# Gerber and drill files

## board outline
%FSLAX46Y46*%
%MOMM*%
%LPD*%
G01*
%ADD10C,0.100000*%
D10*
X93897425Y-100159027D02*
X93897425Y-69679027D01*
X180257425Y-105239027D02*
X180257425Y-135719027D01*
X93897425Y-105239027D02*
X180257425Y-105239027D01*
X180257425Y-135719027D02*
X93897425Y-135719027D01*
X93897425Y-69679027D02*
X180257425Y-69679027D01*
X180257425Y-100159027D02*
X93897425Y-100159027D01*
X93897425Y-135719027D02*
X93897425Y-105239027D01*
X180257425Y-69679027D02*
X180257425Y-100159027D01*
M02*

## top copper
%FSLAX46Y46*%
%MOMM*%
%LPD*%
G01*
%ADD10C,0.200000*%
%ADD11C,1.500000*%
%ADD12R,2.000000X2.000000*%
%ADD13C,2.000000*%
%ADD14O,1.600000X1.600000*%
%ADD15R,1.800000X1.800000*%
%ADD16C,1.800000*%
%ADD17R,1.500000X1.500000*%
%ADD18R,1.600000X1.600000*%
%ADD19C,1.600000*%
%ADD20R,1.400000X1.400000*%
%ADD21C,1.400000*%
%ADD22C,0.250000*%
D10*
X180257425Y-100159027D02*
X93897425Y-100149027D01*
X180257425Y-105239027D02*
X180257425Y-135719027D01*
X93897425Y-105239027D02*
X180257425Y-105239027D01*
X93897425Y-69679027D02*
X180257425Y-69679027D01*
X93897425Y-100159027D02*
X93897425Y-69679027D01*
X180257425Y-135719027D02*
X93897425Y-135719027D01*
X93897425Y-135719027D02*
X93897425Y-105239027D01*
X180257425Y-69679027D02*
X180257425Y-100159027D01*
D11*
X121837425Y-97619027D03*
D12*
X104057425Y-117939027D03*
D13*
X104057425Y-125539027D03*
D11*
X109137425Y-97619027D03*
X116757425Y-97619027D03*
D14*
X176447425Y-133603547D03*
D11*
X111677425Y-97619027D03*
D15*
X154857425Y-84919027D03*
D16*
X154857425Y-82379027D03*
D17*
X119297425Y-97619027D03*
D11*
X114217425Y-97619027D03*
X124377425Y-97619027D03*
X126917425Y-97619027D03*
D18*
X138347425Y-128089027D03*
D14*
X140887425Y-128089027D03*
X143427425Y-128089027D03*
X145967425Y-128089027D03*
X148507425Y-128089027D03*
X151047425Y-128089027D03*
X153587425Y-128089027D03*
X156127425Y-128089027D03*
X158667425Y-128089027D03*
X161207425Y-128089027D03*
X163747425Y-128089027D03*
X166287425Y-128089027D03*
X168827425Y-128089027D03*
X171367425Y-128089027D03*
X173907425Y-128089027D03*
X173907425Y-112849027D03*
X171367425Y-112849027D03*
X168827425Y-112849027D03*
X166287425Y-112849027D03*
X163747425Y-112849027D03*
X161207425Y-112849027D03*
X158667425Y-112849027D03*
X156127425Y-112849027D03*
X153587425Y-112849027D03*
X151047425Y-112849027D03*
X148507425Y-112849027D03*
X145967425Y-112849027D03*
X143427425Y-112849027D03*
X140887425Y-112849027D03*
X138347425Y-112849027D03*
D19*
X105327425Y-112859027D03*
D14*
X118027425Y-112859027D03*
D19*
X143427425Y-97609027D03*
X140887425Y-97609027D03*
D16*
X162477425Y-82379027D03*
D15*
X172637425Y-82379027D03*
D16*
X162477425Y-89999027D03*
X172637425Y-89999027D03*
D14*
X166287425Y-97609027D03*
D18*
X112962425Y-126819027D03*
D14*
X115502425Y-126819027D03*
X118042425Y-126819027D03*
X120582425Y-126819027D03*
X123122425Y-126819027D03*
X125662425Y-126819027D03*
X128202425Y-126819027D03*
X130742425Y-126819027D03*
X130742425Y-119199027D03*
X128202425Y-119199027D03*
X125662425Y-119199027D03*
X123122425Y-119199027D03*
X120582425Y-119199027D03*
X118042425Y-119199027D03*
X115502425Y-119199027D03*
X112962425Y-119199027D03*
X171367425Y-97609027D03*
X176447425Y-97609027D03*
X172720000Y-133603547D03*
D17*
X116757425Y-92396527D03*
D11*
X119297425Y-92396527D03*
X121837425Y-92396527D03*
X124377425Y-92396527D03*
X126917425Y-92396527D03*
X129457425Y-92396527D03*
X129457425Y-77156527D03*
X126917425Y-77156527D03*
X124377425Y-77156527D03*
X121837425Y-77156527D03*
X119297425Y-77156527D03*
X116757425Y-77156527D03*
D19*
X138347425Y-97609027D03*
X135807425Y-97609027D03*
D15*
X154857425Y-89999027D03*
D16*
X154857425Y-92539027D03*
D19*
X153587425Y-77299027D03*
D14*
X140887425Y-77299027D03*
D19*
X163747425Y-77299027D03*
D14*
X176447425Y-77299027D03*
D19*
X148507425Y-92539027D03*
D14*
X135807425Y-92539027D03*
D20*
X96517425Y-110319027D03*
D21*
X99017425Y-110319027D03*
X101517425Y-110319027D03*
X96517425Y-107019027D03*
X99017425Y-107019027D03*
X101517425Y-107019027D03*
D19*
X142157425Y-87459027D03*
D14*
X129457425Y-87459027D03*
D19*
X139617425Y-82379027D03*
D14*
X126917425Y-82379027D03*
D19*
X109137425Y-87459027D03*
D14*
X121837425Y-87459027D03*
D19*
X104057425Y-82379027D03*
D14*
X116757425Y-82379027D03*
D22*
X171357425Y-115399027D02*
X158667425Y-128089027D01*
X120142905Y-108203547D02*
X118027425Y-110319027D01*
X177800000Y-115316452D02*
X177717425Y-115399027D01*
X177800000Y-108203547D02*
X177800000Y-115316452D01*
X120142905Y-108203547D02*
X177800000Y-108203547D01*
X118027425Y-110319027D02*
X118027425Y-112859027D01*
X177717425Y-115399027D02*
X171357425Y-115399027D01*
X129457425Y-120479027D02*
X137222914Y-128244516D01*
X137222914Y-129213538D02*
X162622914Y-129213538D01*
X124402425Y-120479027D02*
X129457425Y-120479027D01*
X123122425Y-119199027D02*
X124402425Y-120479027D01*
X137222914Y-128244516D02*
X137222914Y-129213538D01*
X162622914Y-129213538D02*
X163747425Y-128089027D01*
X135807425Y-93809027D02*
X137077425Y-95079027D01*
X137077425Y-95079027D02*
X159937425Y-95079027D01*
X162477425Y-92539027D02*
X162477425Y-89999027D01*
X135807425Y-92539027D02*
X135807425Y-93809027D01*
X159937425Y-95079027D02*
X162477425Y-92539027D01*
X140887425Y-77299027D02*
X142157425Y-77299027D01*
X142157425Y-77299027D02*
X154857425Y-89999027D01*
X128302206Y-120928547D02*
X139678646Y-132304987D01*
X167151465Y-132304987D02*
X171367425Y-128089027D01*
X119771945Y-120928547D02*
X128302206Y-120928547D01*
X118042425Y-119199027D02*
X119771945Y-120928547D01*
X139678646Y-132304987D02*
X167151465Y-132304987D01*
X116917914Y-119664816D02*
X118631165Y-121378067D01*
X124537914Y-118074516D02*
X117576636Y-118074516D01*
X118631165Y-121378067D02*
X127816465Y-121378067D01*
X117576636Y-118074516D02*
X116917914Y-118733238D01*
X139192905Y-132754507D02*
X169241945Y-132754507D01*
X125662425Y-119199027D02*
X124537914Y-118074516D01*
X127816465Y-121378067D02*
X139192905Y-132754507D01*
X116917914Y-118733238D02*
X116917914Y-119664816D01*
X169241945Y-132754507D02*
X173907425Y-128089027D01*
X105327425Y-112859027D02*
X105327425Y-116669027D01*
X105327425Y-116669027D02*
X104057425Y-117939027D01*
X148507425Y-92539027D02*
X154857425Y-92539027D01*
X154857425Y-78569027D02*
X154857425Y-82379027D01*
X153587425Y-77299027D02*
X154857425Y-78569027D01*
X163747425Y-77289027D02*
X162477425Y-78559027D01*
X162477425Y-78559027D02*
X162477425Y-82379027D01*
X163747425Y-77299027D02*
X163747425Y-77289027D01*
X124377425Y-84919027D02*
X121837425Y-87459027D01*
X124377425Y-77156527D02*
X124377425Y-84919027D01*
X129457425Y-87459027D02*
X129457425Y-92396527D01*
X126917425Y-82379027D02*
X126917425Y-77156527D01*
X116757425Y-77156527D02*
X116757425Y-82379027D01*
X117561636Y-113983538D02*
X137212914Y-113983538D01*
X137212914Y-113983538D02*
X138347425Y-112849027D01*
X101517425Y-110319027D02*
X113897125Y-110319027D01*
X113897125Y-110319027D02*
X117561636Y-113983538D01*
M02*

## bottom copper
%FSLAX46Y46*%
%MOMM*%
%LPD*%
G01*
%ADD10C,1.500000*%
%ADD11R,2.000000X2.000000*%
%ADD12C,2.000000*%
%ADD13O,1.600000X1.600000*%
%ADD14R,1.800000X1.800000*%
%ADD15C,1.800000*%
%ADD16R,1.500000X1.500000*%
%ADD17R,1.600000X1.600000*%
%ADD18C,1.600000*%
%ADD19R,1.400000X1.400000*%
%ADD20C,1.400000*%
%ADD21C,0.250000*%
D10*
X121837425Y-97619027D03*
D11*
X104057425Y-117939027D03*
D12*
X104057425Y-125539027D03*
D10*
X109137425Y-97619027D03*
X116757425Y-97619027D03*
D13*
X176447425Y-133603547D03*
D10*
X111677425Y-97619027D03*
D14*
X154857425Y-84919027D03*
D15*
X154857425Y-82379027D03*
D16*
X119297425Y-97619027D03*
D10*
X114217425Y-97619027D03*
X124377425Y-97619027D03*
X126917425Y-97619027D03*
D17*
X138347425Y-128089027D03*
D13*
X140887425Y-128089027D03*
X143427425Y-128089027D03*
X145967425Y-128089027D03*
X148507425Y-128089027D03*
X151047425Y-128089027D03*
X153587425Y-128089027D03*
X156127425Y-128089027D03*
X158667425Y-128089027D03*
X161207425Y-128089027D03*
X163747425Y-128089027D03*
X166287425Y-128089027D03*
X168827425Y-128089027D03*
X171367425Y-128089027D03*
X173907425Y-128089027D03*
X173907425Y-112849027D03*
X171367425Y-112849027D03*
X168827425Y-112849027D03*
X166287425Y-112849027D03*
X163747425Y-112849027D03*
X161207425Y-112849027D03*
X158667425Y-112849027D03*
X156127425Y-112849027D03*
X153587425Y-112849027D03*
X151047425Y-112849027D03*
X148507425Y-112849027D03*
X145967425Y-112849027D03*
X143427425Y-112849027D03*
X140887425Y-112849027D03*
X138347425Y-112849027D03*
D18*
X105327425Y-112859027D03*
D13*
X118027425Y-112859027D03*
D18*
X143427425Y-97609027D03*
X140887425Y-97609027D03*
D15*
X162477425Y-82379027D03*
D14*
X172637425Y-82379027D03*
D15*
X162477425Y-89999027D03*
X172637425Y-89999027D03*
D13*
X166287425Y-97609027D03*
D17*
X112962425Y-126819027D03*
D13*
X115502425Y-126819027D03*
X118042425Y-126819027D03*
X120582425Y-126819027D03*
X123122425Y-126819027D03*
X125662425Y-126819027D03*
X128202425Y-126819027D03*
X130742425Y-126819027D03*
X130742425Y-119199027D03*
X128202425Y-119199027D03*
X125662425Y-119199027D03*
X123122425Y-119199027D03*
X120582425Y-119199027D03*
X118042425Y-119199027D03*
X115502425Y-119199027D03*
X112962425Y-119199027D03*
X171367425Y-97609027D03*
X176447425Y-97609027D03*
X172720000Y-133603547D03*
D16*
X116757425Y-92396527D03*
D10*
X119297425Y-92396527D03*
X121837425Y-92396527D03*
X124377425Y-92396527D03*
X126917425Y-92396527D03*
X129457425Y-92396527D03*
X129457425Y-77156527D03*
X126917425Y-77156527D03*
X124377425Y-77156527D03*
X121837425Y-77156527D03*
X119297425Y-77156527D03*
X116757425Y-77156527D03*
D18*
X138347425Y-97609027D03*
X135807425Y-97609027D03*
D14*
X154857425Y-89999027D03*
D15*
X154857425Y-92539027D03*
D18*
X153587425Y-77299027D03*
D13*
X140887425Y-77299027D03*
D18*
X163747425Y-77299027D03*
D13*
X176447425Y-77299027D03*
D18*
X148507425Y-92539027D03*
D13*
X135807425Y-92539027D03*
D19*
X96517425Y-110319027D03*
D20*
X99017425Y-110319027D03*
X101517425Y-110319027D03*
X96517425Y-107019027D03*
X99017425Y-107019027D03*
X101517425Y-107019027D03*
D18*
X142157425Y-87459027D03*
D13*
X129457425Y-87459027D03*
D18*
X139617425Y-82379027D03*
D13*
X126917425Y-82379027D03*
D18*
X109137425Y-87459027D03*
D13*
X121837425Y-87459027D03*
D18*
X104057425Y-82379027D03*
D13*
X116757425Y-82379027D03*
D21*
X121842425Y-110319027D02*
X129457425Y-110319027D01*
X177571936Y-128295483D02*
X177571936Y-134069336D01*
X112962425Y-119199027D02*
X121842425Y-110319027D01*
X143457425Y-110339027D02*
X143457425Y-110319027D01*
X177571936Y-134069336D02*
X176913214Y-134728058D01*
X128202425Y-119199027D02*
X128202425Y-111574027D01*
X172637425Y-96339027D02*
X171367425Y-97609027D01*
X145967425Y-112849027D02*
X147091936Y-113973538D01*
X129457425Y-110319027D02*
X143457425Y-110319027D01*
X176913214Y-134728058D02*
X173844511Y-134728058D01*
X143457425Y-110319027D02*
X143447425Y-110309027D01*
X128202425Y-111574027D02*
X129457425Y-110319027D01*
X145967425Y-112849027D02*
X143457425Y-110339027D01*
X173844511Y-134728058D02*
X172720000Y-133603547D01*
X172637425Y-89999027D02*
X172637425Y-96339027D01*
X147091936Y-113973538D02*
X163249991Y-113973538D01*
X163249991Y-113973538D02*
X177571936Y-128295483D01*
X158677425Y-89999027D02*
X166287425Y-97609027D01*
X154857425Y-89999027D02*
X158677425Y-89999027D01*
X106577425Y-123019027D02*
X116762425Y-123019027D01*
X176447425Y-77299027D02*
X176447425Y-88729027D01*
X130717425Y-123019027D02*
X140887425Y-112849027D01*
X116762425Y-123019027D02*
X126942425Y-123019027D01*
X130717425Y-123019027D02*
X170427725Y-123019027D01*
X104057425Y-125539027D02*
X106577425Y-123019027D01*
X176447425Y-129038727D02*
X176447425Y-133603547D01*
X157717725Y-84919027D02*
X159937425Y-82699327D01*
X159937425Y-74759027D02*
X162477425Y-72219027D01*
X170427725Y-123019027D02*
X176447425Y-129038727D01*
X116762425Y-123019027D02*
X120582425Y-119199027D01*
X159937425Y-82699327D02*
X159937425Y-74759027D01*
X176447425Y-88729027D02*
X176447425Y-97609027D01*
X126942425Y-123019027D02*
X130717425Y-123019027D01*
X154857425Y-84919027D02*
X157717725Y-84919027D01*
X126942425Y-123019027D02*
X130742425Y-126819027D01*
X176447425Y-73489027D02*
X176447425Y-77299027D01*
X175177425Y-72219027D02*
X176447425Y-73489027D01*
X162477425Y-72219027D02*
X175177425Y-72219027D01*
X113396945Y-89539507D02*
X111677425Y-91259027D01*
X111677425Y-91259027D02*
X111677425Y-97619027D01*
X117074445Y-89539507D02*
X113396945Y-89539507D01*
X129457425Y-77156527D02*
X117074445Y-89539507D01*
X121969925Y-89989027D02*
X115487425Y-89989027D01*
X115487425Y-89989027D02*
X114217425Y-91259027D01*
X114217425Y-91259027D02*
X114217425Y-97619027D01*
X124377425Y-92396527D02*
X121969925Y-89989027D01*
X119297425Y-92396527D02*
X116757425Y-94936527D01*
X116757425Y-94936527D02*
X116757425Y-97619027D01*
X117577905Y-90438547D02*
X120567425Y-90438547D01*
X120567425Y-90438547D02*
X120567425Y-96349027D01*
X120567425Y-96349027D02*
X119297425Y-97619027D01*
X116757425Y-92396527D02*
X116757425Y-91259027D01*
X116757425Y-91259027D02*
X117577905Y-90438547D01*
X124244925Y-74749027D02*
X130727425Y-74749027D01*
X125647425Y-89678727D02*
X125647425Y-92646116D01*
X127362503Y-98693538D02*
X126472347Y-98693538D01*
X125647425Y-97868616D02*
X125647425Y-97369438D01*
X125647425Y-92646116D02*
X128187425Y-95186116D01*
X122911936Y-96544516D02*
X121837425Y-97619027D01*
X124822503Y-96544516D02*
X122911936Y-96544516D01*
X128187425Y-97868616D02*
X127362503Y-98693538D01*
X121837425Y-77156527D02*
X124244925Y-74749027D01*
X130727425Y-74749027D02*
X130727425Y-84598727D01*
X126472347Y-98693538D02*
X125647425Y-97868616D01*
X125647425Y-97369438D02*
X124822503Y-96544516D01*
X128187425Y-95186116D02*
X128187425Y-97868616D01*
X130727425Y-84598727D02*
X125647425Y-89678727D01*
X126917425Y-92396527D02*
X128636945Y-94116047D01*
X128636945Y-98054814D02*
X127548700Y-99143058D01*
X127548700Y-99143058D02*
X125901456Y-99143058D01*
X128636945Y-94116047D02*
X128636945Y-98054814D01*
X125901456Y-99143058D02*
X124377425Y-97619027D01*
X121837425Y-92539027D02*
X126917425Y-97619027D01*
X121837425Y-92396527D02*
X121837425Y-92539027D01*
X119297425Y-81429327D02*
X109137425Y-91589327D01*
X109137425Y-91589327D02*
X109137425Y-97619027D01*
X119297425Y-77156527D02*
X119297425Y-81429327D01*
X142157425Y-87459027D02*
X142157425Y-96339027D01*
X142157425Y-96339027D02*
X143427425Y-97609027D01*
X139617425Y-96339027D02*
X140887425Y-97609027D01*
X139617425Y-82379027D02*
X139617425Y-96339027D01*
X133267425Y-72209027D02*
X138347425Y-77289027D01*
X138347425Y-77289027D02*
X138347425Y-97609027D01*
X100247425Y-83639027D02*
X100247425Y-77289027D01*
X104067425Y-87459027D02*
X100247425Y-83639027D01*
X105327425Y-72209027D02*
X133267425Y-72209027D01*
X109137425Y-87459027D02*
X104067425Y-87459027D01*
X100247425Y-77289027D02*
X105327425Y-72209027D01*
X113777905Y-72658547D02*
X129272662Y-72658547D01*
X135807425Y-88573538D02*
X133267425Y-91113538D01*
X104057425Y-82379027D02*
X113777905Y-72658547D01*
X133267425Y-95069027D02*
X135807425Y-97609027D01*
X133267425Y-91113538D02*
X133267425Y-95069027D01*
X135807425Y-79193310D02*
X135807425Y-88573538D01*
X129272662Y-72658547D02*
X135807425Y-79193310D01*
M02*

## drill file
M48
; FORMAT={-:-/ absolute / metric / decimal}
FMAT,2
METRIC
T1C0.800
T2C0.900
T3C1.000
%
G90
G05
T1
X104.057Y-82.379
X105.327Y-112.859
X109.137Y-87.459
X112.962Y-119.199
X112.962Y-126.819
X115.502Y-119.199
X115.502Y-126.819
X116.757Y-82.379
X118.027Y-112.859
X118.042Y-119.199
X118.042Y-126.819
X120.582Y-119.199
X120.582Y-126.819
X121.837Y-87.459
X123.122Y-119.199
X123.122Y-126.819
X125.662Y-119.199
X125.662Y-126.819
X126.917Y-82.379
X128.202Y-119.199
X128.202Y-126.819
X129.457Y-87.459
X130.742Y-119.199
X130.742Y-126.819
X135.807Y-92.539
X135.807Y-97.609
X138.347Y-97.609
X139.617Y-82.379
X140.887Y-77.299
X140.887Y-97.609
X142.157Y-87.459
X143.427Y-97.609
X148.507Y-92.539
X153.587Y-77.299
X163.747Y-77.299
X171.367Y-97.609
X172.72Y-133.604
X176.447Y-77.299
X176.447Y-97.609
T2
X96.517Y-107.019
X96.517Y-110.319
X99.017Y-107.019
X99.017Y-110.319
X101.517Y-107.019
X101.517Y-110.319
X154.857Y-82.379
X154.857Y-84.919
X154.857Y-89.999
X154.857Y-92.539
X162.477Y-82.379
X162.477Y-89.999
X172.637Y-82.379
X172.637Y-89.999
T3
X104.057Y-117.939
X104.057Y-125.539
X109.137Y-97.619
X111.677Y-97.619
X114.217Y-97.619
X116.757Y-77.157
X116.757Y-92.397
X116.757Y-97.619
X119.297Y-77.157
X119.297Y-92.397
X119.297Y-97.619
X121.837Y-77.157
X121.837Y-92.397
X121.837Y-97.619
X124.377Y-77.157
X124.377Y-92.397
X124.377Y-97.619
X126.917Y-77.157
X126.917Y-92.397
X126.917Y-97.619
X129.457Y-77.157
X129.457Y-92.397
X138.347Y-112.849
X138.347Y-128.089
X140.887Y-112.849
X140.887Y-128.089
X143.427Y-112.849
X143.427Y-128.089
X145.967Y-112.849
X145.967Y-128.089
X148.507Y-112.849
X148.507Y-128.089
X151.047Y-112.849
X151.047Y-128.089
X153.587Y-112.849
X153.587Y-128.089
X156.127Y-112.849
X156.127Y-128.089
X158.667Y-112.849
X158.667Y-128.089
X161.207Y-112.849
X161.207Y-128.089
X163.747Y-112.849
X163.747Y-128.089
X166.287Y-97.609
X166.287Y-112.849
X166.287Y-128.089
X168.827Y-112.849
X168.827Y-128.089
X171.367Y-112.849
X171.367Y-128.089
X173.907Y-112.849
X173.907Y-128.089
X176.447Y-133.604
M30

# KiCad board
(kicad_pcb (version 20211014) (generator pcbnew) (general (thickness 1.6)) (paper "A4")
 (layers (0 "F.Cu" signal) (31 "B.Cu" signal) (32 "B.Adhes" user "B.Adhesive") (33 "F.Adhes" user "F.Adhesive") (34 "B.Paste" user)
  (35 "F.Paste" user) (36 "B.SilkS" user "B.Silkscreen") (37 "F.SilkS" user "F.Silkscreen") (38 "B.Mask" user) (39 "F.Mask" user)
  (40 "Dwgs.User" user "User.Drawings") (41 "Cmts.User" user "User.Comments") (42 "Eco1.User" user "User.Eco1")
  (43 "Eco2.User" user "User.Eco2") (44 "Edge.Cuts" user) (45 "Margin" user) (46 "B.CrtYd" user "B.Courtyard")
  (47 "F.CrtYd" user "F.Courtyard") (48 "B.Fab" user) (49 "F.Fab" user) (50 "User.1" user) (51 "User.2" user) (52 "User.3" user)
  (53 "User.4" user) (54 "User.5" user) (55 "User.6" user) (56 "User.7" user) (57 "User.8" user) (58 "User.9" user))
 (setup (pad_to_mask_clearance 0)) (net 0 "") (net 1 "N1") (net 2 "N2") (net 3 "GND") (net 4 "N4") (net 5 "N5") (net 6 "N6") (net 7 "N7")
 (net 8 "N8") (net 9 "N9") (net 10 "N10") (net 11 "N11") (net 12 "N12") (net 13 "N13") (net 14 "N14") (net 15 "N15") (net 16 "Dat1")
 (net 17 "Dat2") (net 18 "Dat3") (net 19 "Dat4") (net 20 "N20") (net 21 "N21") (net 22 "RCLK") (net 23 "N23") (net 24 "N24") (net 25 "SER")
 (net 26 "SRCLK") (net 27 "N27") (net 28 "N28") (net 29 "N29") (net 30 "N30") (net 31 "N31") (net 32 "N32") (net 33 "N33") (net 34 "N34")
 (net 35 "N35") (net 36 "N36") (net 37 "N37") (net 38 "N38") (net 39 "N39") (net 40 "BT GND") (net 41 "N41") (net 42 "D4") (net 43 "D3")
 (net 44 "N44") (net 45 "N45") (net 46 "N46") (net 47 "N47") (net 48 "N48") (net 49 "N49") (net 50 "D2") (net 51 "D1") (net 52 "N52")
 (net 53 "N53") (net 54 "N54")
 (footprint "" (layer "F.Cu") (at 121.837425 97.619027)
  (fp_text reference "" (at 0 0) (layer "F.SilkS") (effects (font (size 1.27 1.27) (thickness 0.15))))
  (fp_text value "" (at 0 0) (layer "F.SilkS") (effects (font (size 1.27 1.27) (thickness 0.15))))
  (pad "10" thru_hole circle locked (at 0 0 90) (size 1.5 1.5) (drill 1) (layers *.Cu *.Mask) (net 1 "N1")))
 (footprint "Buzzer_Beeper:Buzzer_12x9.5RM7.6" (layer "F.Cu") (at 104.057425 117.939027 -90)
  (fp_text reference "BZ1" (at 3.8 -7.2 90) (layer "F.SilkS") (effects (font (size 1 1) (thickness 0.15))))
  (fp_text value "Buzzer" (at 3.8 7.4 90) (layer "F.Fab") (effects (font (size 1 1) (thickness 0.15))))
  (pad "1" thru_hole rect locked (at 0 0 270) (size 2 2) (drill 1) (layers *.Cu *.Mask) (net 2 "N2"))
  (pad "2" thru_hole circle locked (at 7.6 0 270) (size 2 2) (drill 1) (layers *.Cu *.Mask) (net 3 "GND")))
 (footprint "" (layer "F.Cu") (at 109.137425 97.619027)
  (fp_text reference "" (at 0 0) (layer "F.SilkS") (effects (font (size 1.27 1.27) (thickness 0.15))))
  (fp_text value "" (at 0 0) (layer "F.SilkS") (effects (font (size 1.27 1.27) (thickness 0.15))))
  (pad "11" thru_hole circle locked (at 0 0 90) (size 1.5 1.5) (drill 1) (layers *.Cu *.Mask) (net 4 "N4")))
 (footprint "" (layer "F.Cu") (at 116.757425 97.619027)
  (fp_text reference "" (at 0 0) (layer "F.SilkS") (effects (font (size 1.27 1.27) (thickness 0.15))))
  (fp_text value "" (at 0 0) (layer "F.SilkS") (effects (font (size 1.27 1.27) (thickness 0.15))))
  (pad "2" thru_hole circle locked (at 0 0 90) (size 1.5 1.5) (drill 1) (layers *.Cu *.Mask) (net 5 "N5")))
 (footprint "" (layer "F.Cu") (at 176.447425 133.603547)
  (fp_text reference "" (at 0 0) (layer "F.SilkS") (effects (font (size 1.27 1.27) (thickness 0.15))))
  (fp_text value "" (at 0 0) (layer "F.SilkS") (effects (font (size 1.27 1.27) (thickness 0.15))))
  (pad "29" thru_hole oval locked (at 0 0 90) (size 1.6 1.6) (drill 1) (layers *.Cu *.Mask) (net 3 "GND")))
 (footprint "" (layer "F.Cu") (at 111.677425 97.619027)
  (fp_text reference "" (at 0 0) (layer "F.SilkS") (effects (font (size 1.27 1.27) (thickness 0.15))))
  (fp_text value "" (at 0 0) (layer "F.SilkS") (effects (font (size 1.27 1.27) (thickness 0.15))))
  (pad "7" thru_hole circle locked (at 0 0 90) (size 1.5 1.5) (drill 1) (layers *.Cu *.Mask) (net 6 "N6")))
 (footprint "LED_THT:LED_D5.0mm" (layer "F.Cu") (at 154.857425 84.919027 90)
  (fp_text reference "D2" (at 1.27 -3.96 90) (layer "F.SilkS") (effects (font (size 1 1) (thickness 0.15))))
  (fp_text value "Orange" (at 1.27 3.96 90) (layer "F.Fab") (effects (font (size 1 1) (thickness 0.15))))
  (pad "1" thru_hole rect locked (at 0 0 90) (size 1.8 1.8) (drill 0.9) (layers *.Cu *.Mask) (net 3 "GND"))
  (pad "2" thru_hole circle locked (at 2.54 0 90) (size 1.8 1.8) (drill 0.9) (layers *.Cu *.Mask) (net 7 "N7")))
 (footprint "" (layer "F.Cu") (at 119.297425 97.619027)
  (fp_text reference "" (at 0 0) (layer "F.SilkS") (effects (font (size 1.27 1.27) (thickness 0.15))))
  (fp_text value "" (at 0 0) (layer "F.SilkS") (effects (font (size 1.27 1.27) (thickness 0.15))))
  (pad "1" thru_hole rect locked (at 0 0 90) (size 1.5 1.5) (drill 1) (layers *.Cu *.Mask) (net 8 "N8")))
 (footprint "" (layer "F.Cu") (at 114.217425 97.619027)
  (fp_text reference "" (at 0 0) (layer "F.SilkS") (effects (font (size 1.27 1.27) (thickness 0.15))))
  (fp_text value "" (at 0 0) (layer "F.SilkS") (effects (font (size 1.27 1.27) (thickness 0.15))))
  (pad "4" thru_hole circle locked (at 0 0 90) (size 1.5 1.5) (drill 1) (layers *.Cu *.Mask) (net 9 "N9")))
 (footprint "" (layer "F.Cu") (at 124.377425 97.619027)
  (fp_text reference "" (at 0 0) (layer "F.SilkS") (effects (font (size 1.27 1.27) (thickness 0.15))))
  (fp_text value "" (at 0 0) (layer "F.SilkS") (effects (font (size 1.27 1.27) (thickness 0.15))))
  (pad "5" thru_hole circle locked (at 0 0 90) (size 1.5 1.5) (drill 1) (layers *.Cu *.Mask) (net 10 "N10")))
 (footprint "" (layer "F.Cu") (at 126.917425 97.619027)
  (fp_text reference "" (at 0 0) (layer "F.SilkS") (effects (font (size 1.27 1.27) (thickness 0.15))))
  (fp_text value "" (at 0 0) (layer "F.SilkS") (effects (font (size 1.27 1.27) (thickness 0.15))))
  (pad "3" thru_hole circle locked (at 0 0 90) (size 1.5 1.5) (drill 1) (layers *.Cu *.Mask) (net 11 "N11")))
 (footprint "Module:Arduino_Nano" (layer "F.Cu") (at 138.347425 128.089027 90)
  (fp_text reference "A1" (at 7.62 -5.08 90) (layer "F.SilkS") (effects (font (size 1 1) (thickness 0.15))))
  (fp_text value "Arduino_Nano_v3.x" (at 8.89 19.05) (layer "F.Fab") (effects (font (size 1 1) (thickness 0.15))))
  (pad "1" thru_hole rect locked (at 0 0 90) (size 1.6 1.6) (drill 1) (layers *.Cu *.Mask) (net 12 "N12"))
  (pad "2" thru_hole oval locked (at 0 2.54 90) (size 1.6 1.6) (drill 1) (layers *.Cu *.Mask) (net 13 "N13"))
  (pad "3" thru_hole oval locked (at 0 5.08 90) (size 1.6 1.6) (drill 1) (layers *.Cu *.Mask) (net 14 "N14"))
  (pad "4" thru_hole oval locked (at 0 7.62 90) (size 1.6 1.6) (drill 1) (layers *.Cu *.Mask) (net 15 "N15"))
  (pad "5" thru_hole oval locked (at 0 10.16 90) (size 1.6 1.6) (drill 1) (layers *.Cu *.Mask) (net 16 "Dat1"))
  (pad "6" thru_hole oval locked (at 0 12.7 90) (size 1.6 1.6) (drill 1) (layers *.Cu *.Mask) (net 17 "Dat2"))
  (pad "7" thru_hole oval locked (at 0 15.24 90) (size 1.6 1.6) (drill 1) (layers *.Cu *.Mask) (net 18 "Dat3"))
  (pad "8" thru_hole oval locked (at 0 17.78 90) (size 1.6 1.6) (drill 1) (layers *.Cu *.Mask) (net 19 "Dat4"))
  (pad "9" thru_hole oval locked (at 0 20.32 90) (size 1.6 1.6) (drill 1) (layers *.Cu *.Mask) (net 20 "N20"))
  (pad "10" thru_hole oval locked (at 0 22.86 90) (size 1.6 1.6) (drill 1) (layers *.Cu *.Mask) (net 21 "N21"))
  (pad "11" thru_hole oval locked (at 0 25.4 90) (size 1.6 1.6) (drill 1) (layers *.Cu *.Mask) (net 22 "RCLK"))
  (pad "12" thru_hole oval locked (at 0 27.94 90) (size 1.6 1.6) (drill 1) (layers *.Cu *.Mask) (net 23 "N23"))
  (pad "13" thru_hole oval locked (at 0 30.48 90) (size 1.6 1.6) (drill 1) (layers *.Cu *.Mask) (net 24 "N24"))
  (pad "14" thru_hole oval locked (at 0 33.02 90) (size 1.6 1.6) (drill 1) (layers *.Cu *.Mask) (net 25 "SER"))
  (pad "15" thru_hole oval locked (at 0 35.56 90) (size 1.6 1.6) (drill 1) (layers *.Cu *.Mask) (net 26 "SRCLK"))
  (pad "16" thru_hole oval locked (at 15.24 35.56 90) (size 1.6 1.6) (drill 1) (layers *.Cu *.Mask) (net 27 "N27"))
  (pad "17" thru_hole oval locked (at 15.24 33.02 90) (size 1.6 1.6) (drill 1) (layers *.Cu *.Mask) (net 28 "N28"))
  (pad "18" thru_hole oval locked (at 15.24 30.48 90) (size 1.6 1.6) (drill 1) (layers *.Cu *.Mask) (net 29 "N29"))
  (pad "19" thru_hole oval locked (at 15.24 27.94 90) (size 1.6 1.6) (drill 1) (layers *.Cu *.Mask) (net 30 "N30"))
  (pad "20" thru_hole oval locked (at 15.24 25.4 90) (size 1.6 1.6) (drill 1) (layers *.Cu *.Mask) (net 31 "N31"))
  (pad "21" thru_hole oval locked (at 15.24 22.86 90) (size 1.6 1.6) (drill 1) (layers *.Cu *.Mask) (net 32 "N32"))
  (pad "22" thru_hole oval locked (at 15.24 20.32 90) (size 1.6 1.6) (drill 1) (layers *.Cu *.Mask) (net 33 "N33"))
  (pad "23" thru_hole oval locked (at 15.24 17.78 90) (size 1.6 1.6) (drill 1) (layers *.Cu *.Mask) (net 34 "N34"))
  (pad "24" thru_hole oval locked (at 15.24 15.24 90) (size 1.6 1.6) (drill 1) (layers *.Cu *.Mask) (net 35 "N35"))
  (pad "25" thru_hole oval locked (at 15.24 12.7 90) (size 1.6 1.6) (drill 1) (layers *.Cu *.Mask) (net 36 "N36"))
  (pad "26" thru_hole oval locked (at 15.24 10.16 90) (size 1.6 1.6) (drill 1) (layers *.Cu *.Mask) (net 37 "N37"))
  (pad "27" thru_hole oval locked (at 15.24 7.62 90) (size 1.6 1.6) (drill 1) (layers *.Cu *.Mask) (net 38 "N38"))
  (pad "28" thru_hole oval locked (at 15.24 5.08 90) (size 1.6 1.6) (drill 1) (layers *.Cu *.Mask) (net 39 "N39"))
  (pad "29" thru_hole oval locked (at 15.24 2.54 90) (size 1.6 1.6) (drill 1) (layers *.Cu *.Mask) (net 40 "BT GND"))
  (pad "30" thru_hole oval locked (at 15.24 0 90) (size 1.6 1.6) (drill 1) (layers *.Cu *.Mask) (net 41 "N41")))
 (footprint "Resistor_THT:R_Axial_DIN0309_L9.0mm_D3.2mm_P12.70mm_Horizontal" (layer "F.Cu") (at 105.327425 112.859027)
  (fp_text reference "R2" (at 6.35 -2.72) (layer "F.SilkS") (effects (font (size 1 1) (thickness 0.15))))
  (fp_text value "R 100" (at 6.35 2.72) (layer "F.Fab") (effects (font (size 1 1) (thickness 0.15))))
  (pad "1" thru_hole circle locked (at 0 0) (size 1.6 1.6) (drill 0.8) (layers *.Cu *.Mask) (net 2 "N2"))
  (pad "2" thru_hole oval locked (at 12.7 0) (size 1.6 1.6) (drill 0.8) (layers *.Cu *.Mask) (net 20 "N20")))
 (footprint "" (layer "F.Cu") (at 143.427425 97.609027)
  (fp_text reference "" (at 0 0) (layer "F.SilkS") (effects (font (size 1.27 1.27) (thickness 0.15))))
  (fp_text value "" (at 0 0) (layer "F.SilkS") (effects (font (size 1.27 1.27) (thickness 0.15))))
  (pad "1" thru_hole circle locked (at 0 0 180) (size 1.6 1.6) (drill 0.8) (layers *.Cu *.Mask) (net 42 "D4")))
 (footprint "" (layer "F.Cu") (at 140.887425 97.609027)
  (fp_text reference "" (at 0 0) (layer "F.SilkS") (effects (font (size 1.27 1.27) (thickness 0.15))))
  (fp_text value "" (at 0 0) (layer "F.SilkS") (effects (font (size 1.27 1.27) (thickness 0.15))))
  (pad "1" thru_hole circle locked (at 0 0 180) (size 1.6 1.6) (drill 0.8) (layers *.Cu *.Mask) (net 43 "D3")))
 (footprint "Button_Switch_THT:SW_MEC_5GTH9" (layer "F.Cu") (at 172.637425 82.379027 -90)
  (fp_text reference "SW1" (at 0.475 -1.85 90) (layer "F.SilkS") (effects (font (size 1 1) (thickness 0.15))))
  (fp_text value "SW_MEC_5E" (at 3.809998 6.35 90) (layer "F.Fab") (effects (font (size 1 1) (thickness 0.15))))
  (pad "1" thru_hole circle locked (at 0 10.16) (size 1.8 1.8) (drill 0.9) (layers *.Cu *.Mask) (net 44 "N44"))
  (pad "1" thru_hole rect locked (at 0 0) (size 1.8 1.8) (drill 0.9) (layers *.Cu *.Mask) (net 44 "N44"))
  (pad "2" thru_hole circle locked (at 7.62 10.16) (size 1.8 1.8) (drill 0.9) (layers *.Cu *.Mask) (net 38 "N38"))
  (pad "2" thru_hole circle locked (at 7.62 0) (size 1.8 1.8) (drill 0.9) (layers *.Cu *.Mask) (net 38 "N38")))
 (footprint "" (layer "F.Cu") (at 166.287425 97.609027)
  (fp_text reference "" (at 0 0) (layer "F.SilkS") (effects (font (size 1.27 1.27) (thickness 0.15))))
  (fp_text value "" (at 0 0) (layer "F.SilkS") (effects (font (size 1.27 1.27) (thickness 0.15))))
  (pad "12" thru_hole oval locked (at 0 0 90) (size 1.6 1.6) (drill 1) (layers *.Cu *.Mask) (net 23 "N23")))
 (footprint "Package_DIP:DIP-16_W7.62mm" (layer "F.Cu") (at 112.962425 126.819027 90)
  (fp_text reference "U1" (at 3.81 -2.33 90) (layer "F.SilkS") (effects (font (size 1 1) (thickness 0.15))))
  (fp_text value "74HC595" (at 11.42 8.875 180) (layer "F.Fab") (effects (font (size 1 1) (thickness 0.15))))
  (pad "1" thru_hole rect locked (at 0 0 90) (size 1.6 1.6) (drill 0.8) (layers *.Cu *.Mask) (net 6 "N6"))
  (pad "2" thru_hole oval locked (at 0 2.54 90) (size 1.6 1.6) (drill 0.8) (layers *.Cu *.Mask) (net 9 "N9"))
  (pad "3" thru_hole oval locked (at 0 5.08 90) (size 1.6 1.6) (drill 0.8) (layers *.Cu *.Mask) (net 5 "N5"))
  (pad "4" thru_hole oval locked (at 0 7.62 90) (size 1.6 1.6) (drill 0.8) (layers *.Cu *.Mask) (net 8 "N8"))
  (pad "5" thru_hole oval locked (at 0 10.16 90) (size 1.6 1.6) (drill 0.8) (layers *.Cu *.Mask) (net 1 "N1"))
  (pad "6" thru_hole oval locked (at 0 12.7 90) (size 1.6 1.6) (drill 0.8) (layers *.Cu *.Mask) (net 10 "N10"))
  (pad "7" thru_hole oval locked (at 0 15.24 90) (size 1.6 1.6) (drill 0.8) (layers *.Cu *.Mask) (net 11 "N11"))
  (pad "8" thru_hole oval locked (at 0 17.78 90) (size 1.6 1.6) (drill 0.8) (layers *.Cu *.Mask) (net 3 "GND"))
  (pad "9" thru_hole oval locked (at 7.62 17.78 90) (size 1.6 1.6) (drill 0.8) (layers *.Cu *.Mask) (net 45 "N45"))
  (pad "10" thru_hole oval locked (at 7.62 15.24 90) (size 1.6 1.6) (drill 0.8) (layers *.Cu *.Mask) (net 38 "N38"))
  (pad "11" thru_hole oval locked (at 7.62 12.7 90) (size 1.6 1.6) (drill 0.8) (layers *.Cu *.Mask) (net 26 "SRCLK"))
  (pad "12" thru_hole oval locked (at 7.62 10.16 90) (size 1.6 1.6) (drill 0.8) (layers *.Cu *.Mask) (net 22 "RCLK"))
  (pad "13" thru_hole oval locked (at 7.62 7.62 90) (size 1.6 1.6) (drill 0.8) (layers *.Cu *.Mask) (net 3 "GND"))
  (pad "14" thru_hole oval locked (at 7.62 5.08 90) (size 1.6 1.6) (drill 0.8) (layers *.Cu *.Mask) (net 25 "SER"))
  (pad "15" thru_hole oval locked (at 7.62 2.54 90) (size 1.6 1.6) (drill 0.8) (layers *.Cu *.Mask) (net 4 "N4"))
  (pad "16" thru_hole oval locked (at 7.62 0 90) (size 1.6 1.6) (drill 0.8) (layers *.Cu *.Mask) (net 38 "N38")))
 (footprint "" (layer "F.Cu") (at 171.367425 97.609027)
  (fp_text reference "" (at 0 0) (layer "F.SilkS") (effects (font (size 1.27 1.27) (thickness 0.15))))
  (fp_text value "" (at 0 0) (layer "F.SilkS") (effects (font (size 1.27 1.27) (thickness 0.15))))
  (pad "2" thru_hole oval locked (at 0 0 180) (size 1.6 1.6) (drill 0.8) (layers *.Cu *.Mask) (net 38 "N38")))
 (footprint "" (layer "F.Cu") (at 176.447425 97.609027)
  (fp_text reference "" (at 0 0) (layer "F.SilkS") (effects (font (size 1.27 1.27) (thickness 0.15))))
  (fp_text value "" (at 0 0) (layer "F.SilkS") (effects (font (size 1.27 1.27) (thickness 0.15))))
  (pad "2" thru_hole oval locked (at 0 0) (size 1.6 1.6) (drill 0.8) (layers *.Cu *.Mask) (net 3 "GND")))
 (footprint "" (layer "F.Cu") (at 172.72 133.603547)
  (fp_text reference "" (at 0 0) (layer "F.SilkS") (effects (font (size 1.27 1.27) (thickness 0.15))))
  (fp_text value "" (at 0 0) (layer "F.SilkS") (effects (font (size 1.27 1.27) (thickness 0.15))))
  (pad "2" thru_hole oval locked (at 0 0 180) (size 1.6 1.6) (drill 0.8) (layers *.Cu *.Mask) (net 38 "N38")))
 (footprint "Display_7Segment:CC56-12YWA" (layer "F.Cu") (at 116.757425 92.396527 90)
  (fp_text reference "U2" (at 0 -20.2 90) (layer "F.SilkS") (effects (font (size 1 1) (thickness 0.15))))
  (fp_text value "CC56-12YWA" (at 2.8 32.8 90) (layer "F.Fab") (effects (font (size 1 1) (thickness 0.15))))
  (pad "1" thru_hole rect locked (at 0 0 90) (size 1.5 1.5) (drill 1) (layers *.Cu *.Mask) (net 8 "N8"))
  (pad "2" thru_hole circle locked (at 0 2.54 90) (size 1.5 1.5) (drill 1) (layers *.Cu *.Mask) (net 5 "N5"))
  (pad "3" thru_hole circle locked (at 0 5.08 90) (size 1.5 1.5) (drill 1) (layers *.Cu *.Mask) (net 11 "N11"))
  (pad "4" thru_hole circle locked (at 0 7.62 90) (size 1.5 1.5) (drill 1) (layers *.Cu *.Mask) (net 9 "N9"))
  (pad "5" thru_hole circle locked (at 0 10.16 90) (size 1.5 1.5) (drill 1) (layers *.Cu *.Mask) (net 10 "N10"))
  (pad "6" thru_hole circle locked (at 0 12.7 90) (size 1.5 1.5) (drill 1) (layers *.Cu *.Mask) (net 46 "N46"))
  (pad "7" thru_hole circle locked (at 15.24 12.7 90) (size 1.5 1.5) (drill 1) (layers *.Cu *.Mask) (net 6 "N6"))
  (pad "8" thru_hole circle locked (at 15.24 10.16 90) (size 1.5 1.5) (drill 1) (layers *.Cu *.Mask) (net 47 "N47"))
  (pad "9" thru_hole circle locked (at 15.24 7.62 90) (size 1.5 1.5) (drill 1) (layers *.Cu *.Mask) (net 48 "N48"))
  (pad "10" thru_hole circle locked (at 15.24 5.08 90) (size 1.5 1.5) (drill 1) (layers *.Cu *.Mask) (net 1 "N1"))
  (pad "11" thru_hole circle locked (at 15.24 2.54 90) (size 1.5 1.5) (drill 1) (layers *.Cu *.Mask) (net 4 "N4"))
  (pad "12" thru_hole circle locked (at 15.24 0 90) (size 1.5 1.5) (drill 1) (layers *.Cu *.Mask) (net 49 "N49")))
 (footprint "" (layer "F.Cu") (at 138.347425 97.609027)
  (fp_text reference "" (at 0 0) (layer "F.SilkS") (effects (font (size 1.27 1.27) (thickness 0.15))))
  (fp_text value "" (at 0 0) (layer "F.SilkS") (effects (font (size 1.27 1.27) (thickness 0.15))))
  (pad "1" thru_hole circle locked (at 0 0) (size 1.6 1.6) (drill 0.8) (layers *.Cu *.Mask) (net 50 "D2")))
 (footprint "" (layer "F.Cu") (at 135.807425 97.609027)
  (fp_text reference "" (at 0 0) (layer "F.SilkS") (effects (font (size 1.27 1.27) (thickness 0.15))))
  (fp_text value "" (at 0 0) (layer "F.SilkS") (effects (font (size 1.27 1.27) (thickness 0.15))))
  (pad "1" thru_hole circle locked (at 0 0) (size 1.6 1.6) (drill 0.8) (layers *.Cu *.Mask) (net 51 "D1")))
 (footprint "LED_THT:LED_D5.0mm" (layer "F.Cu") (at 154.857425 89.999027 -90)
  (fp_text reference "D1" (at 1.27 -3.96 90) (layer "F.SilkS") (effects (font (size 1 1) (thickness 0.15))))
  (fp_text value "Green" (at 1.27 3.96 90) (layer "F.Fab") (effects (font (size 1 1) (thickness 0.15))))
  (pad "1" thru_hole rect locked (at 0 0 270) (size 1.8 1.8) (drill 0.9) (layers *.Cu *.Mask) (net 23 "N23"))
  (pad "2" thru_hole circle locked (at 2.54 0 270) (size 1.8 1.8) (drill 0.9) (layers *.Cu *.Mask) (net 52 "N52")))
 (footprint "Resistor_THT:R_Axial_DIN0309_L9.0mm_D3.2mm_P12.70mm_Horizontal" (layer "B.Cu") (at 153.587425 77.299027 180)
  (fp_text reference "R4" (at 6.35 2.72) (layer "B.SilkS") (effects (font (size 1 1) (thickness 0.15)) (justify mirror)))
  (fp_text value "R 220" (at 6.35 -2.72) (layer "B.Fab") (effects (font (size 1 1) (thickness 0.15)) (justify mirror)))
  (pad "1" thru_hole circle locked (at 0 0 180) (size 1.6 1.6) (drill 0.8) (layers *.Cu *.Mask) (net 7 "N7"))
  (pad "2" thru_hole oval locked (at 12.7 0 180) (size 1.6 1.6) (drill 0.8) (layers *.Cu *.Mask) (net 23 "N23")))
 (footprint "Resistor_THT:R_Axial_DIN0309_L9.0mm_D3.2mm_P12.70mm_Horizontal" (layer "B.Cu") (at 163.747425 77.299027)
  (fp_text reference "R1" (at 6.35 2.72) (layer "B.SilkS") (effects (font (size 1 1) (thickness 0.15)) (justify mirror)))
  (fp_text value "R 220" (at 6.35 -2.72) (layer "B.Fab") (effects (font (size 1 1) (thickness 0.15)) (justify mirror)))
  (pad "1" thru_hole circle locked (at 0 0) (size 1.6 1.6) (drill 0.8) (layers *.Cu *.Mask) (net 44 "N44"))
  (pad "2" thru_hole oval locked (at 12.7 0) (size 1.6 1.6) (drill 0.8) (layers *.Cu *.Mask) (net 3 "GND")))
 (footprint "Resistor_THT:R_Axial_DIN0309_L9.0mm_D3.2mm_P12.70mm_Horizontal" (layer "B.Cu") (at 148.507425 92.539027 180)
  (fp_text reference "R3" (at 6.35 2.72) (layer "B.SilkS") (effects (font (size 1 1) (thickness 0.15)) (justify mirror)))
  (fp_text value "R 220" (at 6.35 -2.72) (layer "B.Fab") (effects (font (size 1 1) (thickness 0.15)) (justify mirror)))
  (pad "1" thru_hole circle locked (at 0 0 180) (size 1.6 1.6) (drill 0.8) (layers *.Cu *.Mask) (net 52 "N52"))
  (pad "2" thru_hole oval locked (at 12.7 0 180) (size 1.6 1.6) (drill 0.8) (layers *.Cu *.Mask) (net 38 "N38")))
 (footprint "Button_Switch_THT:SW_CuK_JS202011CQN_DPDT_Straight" (layer "B.Cu") (at 96.517425 110.319027)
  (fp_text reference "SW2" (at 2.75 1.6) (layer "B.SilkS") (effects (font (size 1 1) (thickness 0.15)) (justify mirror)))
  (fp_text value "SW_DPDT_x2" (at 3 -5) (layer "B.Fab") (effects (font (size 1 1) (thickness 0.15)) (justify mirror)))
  (pad "1" thru_hole rect locked (at 0 0) (size 1.4 1.4) (drill 0.9) (layers *.Cu *.Mask) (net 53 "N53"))
  (pad "2" thru_hole circle locked (at 2.5 0) (size 1.4 1.4) (drill 0.9) (layers *.Cu *.Mask) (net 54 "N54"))
  (pad "3" thru_hole circle locked (at 5 0) (size 1.4 1.4) (drill 0.9) (layers *.Cu *.Mask) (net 41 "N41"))
  (pad "4" thru_hole circle locked (at 0 -3.3) (size 1.4 1.4) (drill 0.9) (layers *.Cu *.Mask))
  (pad "5" thru_hole circle locked (at 2.5 -3.3) (size 1.4 1.4) (drill 0.9) (layers *.Cu *.Mask))
  (pad "6" thru_hole circle locked (at 5 -3.3) (size 1.4 1.4) (drill 0.9) (layers *.Cu *.Mask)))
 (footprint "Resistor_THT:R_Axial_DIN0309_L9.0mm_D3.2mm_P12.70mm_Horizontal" (layer "B.Cu") (at 142.157425 87.459027 180)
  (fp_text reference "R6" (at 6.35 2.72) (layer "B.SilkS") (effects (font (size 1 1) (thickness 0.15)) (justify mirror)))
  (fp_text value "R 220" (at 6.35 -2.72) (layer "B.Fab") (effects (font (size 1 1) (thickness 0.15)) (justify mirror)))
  (pad "1" thru_hole circle locked (at 0 0 180) (size 1.6 1.6) (drill 0.8) (layers *.Cu *.Mask) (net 19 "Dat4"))
  (pad "2" thru_hole oval locked (at 12.7 0 180) (size 1.6 1.6) (drill 0.8) (layers *.Cu *.Mask) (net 46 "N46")))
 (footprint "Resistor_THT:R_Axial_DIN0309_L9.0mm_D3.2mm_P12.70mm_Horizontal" (layer "B.Cu") (at 139.617425 82.379027 180)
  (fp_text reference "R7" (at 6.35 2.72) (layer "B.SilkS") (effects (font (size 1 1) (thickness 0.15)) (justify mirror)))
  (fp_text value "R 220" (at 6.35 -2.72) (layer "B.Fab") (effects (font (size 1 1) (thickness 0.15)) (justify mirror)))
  (pad "1" thru_hole circle locked (at 0 0 180) (size 1.6 1.6) (drill 0.8) (layers *.Cu *.Mask) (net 18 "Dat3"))
  (pad "2" thru_hole oval locked (at 12.7 0 180) (size 1.6 1.6) (drill 0.8) (layers *.Cu *.Mask) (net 47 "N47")))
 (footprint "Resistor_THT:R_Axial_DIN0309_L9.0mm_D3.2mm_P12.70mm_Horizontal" (layer "B.Cu") (at 109.137425 87.459027)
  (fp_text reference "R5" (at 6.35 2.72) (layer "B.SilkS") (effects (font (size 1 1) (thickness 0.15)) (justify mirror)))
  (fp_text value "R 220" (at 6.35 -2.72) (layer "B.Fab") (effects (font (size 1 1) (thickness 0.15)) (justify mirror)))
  (pad "1" thru_hole circle locked (at 0 0) (size 1.6 1.6) (drill 0.8) (layers *.Cu *.Mask) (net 17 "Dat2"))
  (pad "2" thru_hole oval locked (at 12.7 0) (size 1.6 1.6) (drill 0.8) (layers *.Cu *.Mask) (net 48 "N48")))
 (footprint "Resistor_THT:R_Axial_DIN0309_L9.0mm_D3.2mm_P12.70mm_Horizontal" (layer "B.Cu") (at 104.057425 82.379027)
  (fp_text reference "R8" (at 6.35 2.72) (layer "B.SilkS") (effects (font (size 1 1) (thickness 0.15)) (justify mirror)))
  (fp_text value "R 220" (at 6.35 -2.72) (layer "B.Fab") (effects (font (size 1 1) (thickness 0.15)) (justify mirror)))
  (pad "1" thru_hole circle locked (at 0 0) (size 1.6 1.6) (drill 0.8) (layers *.Cu *.Mask) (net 16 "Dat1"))
  (pad "2" thru_hole oval locked (at 12.7 0) (size 1.6 1.6) (drill 0.8) (layers *.Cu *.Mask) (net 49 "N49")))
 (gr_line (start 180.257425 100.159027) (end 93.897425 100.149027) (layer "F.Cu") (width 0.2))
 (gr_line (start 180.257425 105.239027) (end 180.257425 135.719027) (layer "F.Cu") (width 0.2))
 (gr_line (start 93.897425 105.239027) (end 180.257425 105.239027) (layer "F.Cu") (width 0.2))
 (gr_line (start 93.897425 69.679027) (end 180.257425 69.679027) (layer "F.Cu") (width 0.2))
 (gr_line (start 93.897425 100.159027) (end 93.897425 69.679027) (layer "F.Cu") (width 0.2))
 (gr_line (start 180.257425 135.719027) (end 93.897425 135.719027) (layer "F.Cu") (width 0.2))
 (gr_line (start 93.897425 135.719027) (end 93.897425 105.239027) (layer "F.Cu") (width 0.2))
 (gr_line (start 180.257425 69.679027) (end 180.257425 100.159027) (layer "F.Cu") (width 0.2))
 (gr_line (start 93.897425 100.159027) (end 93.897425 69.679027) (layer "Edge.Cuts") (width 0.1))
 (gr_line (start 180.257425 105.239027) (end 180.257425 135.719027) (layer "Edge.Cuts") (width 0.1))
 (gr_line (start 93.897425 105.239027) (end 180.257425 105.239027) (layer "Edge.Cuts") (width 0.1))
 (gr_line (start 180.257425 135.719027) (end 93.897425 135.719027) (layer "Edge.Cuts") (width 0.1))
 (gr_line (start 93.897425 69.679027) (end 180.257425 69.679027) (layer "Edge.Cuts") (width 0.1))
 (gr_line (start 180.257425 100.159027) (end 93.897425 100.159027) (layer "Edge.Cuts") (width 0.1))
 (gr_line (start 93.897425 135.719027) (end 93.897425 105.239027) (layer "Edge.Cuts") (width 0.1))
 (gr_line (start 180.257425 69.679027) (end 180.257425 100.159027) (layer "Edge.Cuts") (width 0.1))
 (segment (start 171.357425 115.399027) (end 158.667425 128.089027) (width 0.25) (layer "F.Cu") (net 20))
 (segment (start 120.142905 108.203547) (end 118.027425 110.319027) (width 0.25) (layer "F.Cu") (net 20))
 (segment (start 177.8 115.316452) (end 177.717425 115.399027) (width 0.25) (layer "F.Cu") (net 20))
 (segment (start 177.8 108.203547) (end 177.8 115.316452) (width 0.25) (layer "F.Cu") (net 20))
 (segment (start 120.142905 108.203547) (end 177.8 108.203547) (width 0.25) (layer "F.Cu") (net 20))
 (segment (start 118.027425 110.319027) (end 118.027425 112.859027) (width 0.25) (layer "F.Cu") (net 20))
 (segment (start 177.717425 115.399027) (end 171.357425 115.399027) (width 0.25) (layer "F.Cu") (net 20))
 (segment (start 129.457425 120.479027) (end 137.222914 128.244516) (width 0.25) (layer "F.Cu") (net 22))
 (segment (start 137.222914 129.213538) (end 162.622914 129.213538) (width 0.25) (layer "F.Cu") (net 22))
 (segment (start 124.402425 120.479027) (end 129.457425 120.479027) (width 0.25) (layer "F.Cu") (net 22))
 (segment (start 123.122425 119.199027) (end 124.402425 120.479027) (width 0.25) (layer "F.Cu") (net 22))
 (segment (start 137.222914 128.244516) (end 137.222914 129.213538) (width 0.25) (layer "F.Cu") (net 22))
 (segment (start 162.622914 129.213538) (end 163.747425 128.089027) (width 0.25) (layer "F.Cu") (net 22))
 (segment (start 135.807425 93.809027) (end 137.077425 95.079027) (width 0.25) (layer "F.Cu") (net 38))
 (segment (start 137.077425 95.079027) (end 159.937425 95.079027) (width 0.25) (layer "F.Cu") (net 38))
 (segment (start 162.477425 92.539027) (end 162.477425 89.999027) (width 0.25) (layer "F.Cu") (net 38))
 (segment (start 135.807425 92.539027) (end 135.807425 93.809027) (width 0.25) (layer "F.Cu") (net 38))
 (segment (start 159.937425 95.079027) (end 162.477425 92.539027) (width 0.25) (layer "F.Cu") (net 38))
 (segment (start 121.842425 110.319027) (end 129.457425 110.319027) (width 0.25) (layer "B.Cu") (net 38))
 (segment (start 177.571936 128.295483) (end 177.571936 134.069336) (width 0.25) (layer "B.Cu") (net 38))
 (segment (start 112.962425 119.199027) (end 121.842425 110.319027) (width 0.25) (layer "B.Cu") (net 38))
 (segment (start 143.457425 110.339027) (end 143.457425 110.319027) (width 0.25) (layer "B.Cu") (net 38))
 (segment (start 177.571936 134.069336) (end 176.913214 134.728058) (width 0.25) (layer "B.Cu") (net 38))
 (segment (start 128.202425 119.199027) (end 128.202425 111.574027) (width 0.25) (layer "B.Cu") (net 38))
 (segment (start 172.637425 96.339027) (end 171.367425 97.609027) (width 0.25) (layer "B.Cu") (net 38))
 (segment (start 145.967425 112.849027) (end 147.091936 113.973538) (width 0.25) (layer "B.Cu") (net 38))
 (segment (start 129.457425 110.319027) (end 143.457425 110.319027) (width 0.25) (layer "B.Cu") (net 38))
 (segment (start 176.913214 134.728058) (end 173.844511 134.728058) (width 0.25) (layer "B.Cu") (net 38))
 (segment (start 143.457425 110.319027) (end 143.447425 110.309027) (width 0.25) (layer "B.Cu") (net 38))
 (segment (start 128.202425 111.574027) (end 129.457425 110.319027) (width 0.25) (layer "B.Cu") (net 38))
 (segment (start 145.967425 112.849027) (end 143.457425 110.339027) (width 0.25) (layer "B.Cu") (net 38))
 (segment (start 173.844511 134.728058) (end 172.72 133.603547) (width 0.25) (layer "B.Cu") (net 38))
 (segment (start 172.637425 89.999027) (end 172.637425 96.339027) (width 0.25) (layer "B.Cu") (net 38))
 (segment (start 147.091936 113.973538) (end 163.249991 113.973538) (width 0.25) (layer "B.Cu") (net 38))
 (segment (start 163.249991 113.973538) (end 177.571936 128.295483) (width 0.25) (layer "B.Cu") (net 38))
 (segment (start 140.887425 77.299027) (end 142.157425 77.299027) (width 0.25) (layer "F.Cu") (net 23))
 (segment (start 142.157425 77.299027) (end 154.857425 89.999027) (width 0.25) (layer "F.Cu") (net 23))
 (segment (start 158.677425 89.999027) (end 166.287425 97.609027) (width 0.25) (layer "B.Cu") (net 23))
 (segment (start 154.857425 89.999027) (end 158.677425 89.999027) (width 0.25) (layer "B.Cu") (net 23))
 (segment (start 106.577425 123.019027) (end 116.762425 123.019027) (width 0.25) (layer "B.Cu") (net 3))
 (segment (start 176.447425 77.299027) (end 176.447425 88.729027) (width 0.25) (layer "B.Cu") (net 3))
 (segment (start 130.717425 123.019027) (end 140.887425 112.849027) (width 0.25) (layer "B.Cu") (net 3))
 (segment (start 116.762425 123.019027) (end 126.942425 123.019027) (width 0.25) (layer "B.Cu") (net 3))
 (segment (start 130.717425 123.019027) (end 170.427725 123.019027) (width 0.25) (layer "B.Cu") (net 3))
 (segment (start 104.057425 125.539027) (end 106.577425 123.019027) (width 0.25) (layer "B.Cu") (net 3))
 (segment (start 176.447425 129.038727) (end 176.447425 133.603547) (width 0.25) (layer "B.Cu") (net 3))
 (segment (start 157.717725 84.919027) (end 159.937425 82.699327) (width 0.25) (layer "B.Cu") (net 3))
 (segment (start 159.937425 74.759027) (end 162.477425 72.219027) (width 0.25) (layer "B.Cu") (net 3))
 (segment (start 170.427725 123.019027) (end 176.447425 129.038727) (width 0.25) (layer "B.Cu") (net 3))
 (segment (start 116.762425 123.019027) (end 120.582425 119.199027) (width 0.25) (layer "B.Cu") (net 3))
 (segment (start 159.937425 82.699327) (end 159.937425 74.759027) (width 0.25) (layer "B.Cu") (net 3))
 (segment (start 176.447425 88.729027) (end 176.447425 97.609027) (width 0.25) (layer "B.Cu") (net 3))
 (segment (start 126.942425 123.019027) (end 130.717425 123.019027) (width 0.25) (layer "B.Cu") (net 3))
 (segment (start 154.857425 84.919027) (end 157.717725 84.919027) (width 0.25) (layer "B.Cu") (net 3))
 (segment (start 126.942425 123.019027) (end 130.742425 126.819027) (width 0.25) (layer "B.Cu") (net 3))
 (segment (start 176.447425 73.489027) (end 176.447425 77.299027) (width 0.25) (layer "B.Cu") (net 3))
 (segment (start 175.177425 72.219027) (end 176.447425 73.489027) (width 0.25) (layer "B.Cu") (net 3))
 (segment (start 162.477425 72.219027) (end 175.177425 72.219027) (width 0.25) (layer "B.Cu") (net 3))
 (segment (start 128.302206 120.928547) (end 139.678646 132.304987) (width 0.25) (layer "F.Cu") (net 25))
 (segment (start 167.151465 132.304987) (end 171.367425 128.089027) (width 0.25) (layer "F.Cu") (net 25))
 (segment (start 119.771945 120.928547) (end 128.302206 120.928547) (width 0.25) (layer "F.Cu") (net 25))
 (segment (start 118.042425 119.199027) (end 119.771945 120.928547) (width 0.25) (layer "F.Cu") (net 25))
 (segment (start 139.678646 132.304987) (end 167.151465 132.304987) (width 0.25) (layer "F.Cu") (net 25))
 (segment (start 116.917914 119.664816) (end 118.631165 121.378067) (width 0.25) (layer "F.Cu") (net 26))
 (segment (start 124.537914 118.074516) (end 117.576636 118.074516) (width 0.25) (layer "F.Cu") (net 26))
 (segment (start 118.631165 121.378067) (end 127.816465 121.378067) (width 0.25) (layer "F.Cu") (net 26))
 (segment (start 117.576636 118.074516) (end 116.917914 118.733238) (width 0.25) (layer "F.Cu") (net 26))
 (segment (start 139.192905 132.754507) (end 169.241945 132.754507) (width 0.25) (layer "F.Cu") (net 26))
 (segment (start 125.662425 119.199027) (end 124.537914 118.074516) (width 0.25) (layer "F.Cu") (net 26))
 (segment (start 127.816465 121.378067) (end 139.192905 132.754507) (width 0.25) (layer "F.Cu") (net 26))
 (segment (start 116.917914 118.733238) (end 116.917914 119.664816) (width 0.25) (layer "F.Cu") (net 26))
 (segment (start 169.241945 132.754507) (end 173.907425 128.089027) (width 0.25) (layer "F.Cu") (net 26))
 (segment (start 105.327425 112.859027) (end 105.327425 116.669027) (width 0.25) (layer "F.Cu") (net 2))
 (segment (start 105.327425 116.669027) (end 104.057425 117.939027) (width 0.25) (layer "F.Cu") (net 2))
 (segment (start 148.507425 92.539027) (end 154.857425 92.539027) (width 0.25) (layer "F.Cu") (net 52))
 (segment (start 154.857425 78.569027) (end 154.857425 82.379027) (width 0.25) (layer "F.Cu") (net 7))
 (segment (start 153.587425 77.299027) (end 154.857425 78.569027) (width 0.25) (layer "F.Cu") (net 7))
 (segment (start 163.747425 77.289027) (end 162.477425 78.559027) (width 0.25) (layer "F.Cu") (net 44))
 (segment (start 162.477425 78.559027) (end 162.477425 82.379027) (width 0.25) (layer "F.Cu") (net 44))
 (segment (start 163.747425 77.299027) (end 163.747425 77.289027) (width 0.25) (layer "F.Cu") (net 44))
 (segment (start 113.396945 89.539507) (end 111.677425 91.259027) (width 0.25) (layer "B.Cu") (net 6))
 (segment (start 111.677425 91.259027) (end 111.677425 97.619027) (width 0.25) (layer "B.Cu") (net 6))
 (segment (start 117.074445 89.539507) (end 113.396945 89.539507) (width 0.25) (layer "B.Cu") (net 6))
 (segment (start 129.457425 77.156527) (end 117.074445 89.539507) (width 0.25) (layer "B.Cu") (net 6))
 (segment (start 121.969925 89.989027) (end 115.487425 89.989027) (width 0.25) (layer "B.Cu") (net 9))
 (segment (start 115.487425 89.989027) (end 114.217425 91.259027) (width 0.25) (layer "B.Cu") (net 9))
 (segment (start 114.217425 91.259027) (end 114.217425 97.619027) (width 0.25) (layer "B.Cu") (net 9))
 (segment (start 124.377425 92.396527) (end 121.969925 89.989027) (width 0.25) (layer "B.Cu") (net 9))
 (segment (start 119.297425 92.396527) (end 116.757425 94.936527) (width 0.25) (layer "B.Cu") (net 5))
 (segment (start 116.757425 94.936527) (end 116.757425 97.619027) (width 0.25) (layer "B.Cu") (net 5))
 (segment (start 117.577905 90.438547) (end 120.567425 90.438547) (width 0.25) (layer "B.Cu") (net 8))
 (segment (start 120.567425 90.438547) (end 120.567425 96.349027) (width 0.25) (layer "B.Cu") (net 8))
 (segment (start 120.567425 96.349027) (end 119.297425 97.619027) (width 0.25) (layer "B.Cu") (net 8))
 (segment (start 116.757425 92.396527) (end 116.757425 91.259027) (width 0.25) (layer "B.Cu") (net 8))
 (segment (start 116.757425 91.259027) (end 117.577905 90.438547) (width 0.25) (layer "B.Cu") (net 8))
 (segment (start 124.244925 74.749027) (end 130.727425 74.749027) (width 0.25) (layer "B.Cu") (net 1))
 (segment (start 125.647425 89.678727) (end 125.647425 92.646116) (width 0.25) (layer "B.Cu") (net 1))
 (segment (start 127.362503 98.693538) (end 126.472347 98.693538) (width 0.25) (layer "B.Cu") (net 1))
 (segment (start 125.647425 97.868616) (end 125.647425 97.369438) (width 0.25) (layer "B.Cu") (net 1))
 (segment (start 125.647425 92.646116) (end 128.187425 95.186116) (width 0.25) (layer "B.Cu") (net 1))
 (segment (start 122.911936 96.544516) (end 121.837425 97.619027) (width 0.25) (layer "B.Cu") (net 1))
 (segment (start 124.822503 96.544516) (end 122.911936 96.544516) (width 0.25) (layer "B.Cu") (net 1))
 (segment (start 128.187425 97.868616) (end 127.362503 98.693538) (width 0.25) (layer "B.Cu") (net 1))
 (segment (start 121.837425 77.156527) (end 124.244925 74.749027) (width 0.25) (layer "B.Cu") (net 1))
 (segment (start 130.727425 74.749027) (end 130.727425 84.598727) (width 0.25) (layer "B.Cu") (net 1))
 (segment (start 126.472347 98.693538) (end 125.647425 97.868616) (width 0.25) (layer "B.Cu") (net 1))
 (segment (start 125.647425 97.369438) (end 124.822503 96.544516) (width 0.25) (layer "B.Cu") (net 1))
 (segment (start 128.187425 95.186116) (end 128.187425 97.868616) (width 0.25) (layer "B.Cu") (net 1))
 (segment (start 130.727425 84.598727) (end 125.647425 89.678727) (width 0.25) (layer "B.Cu") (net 1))
 (segment (start 126.917425 92.396527) (end 128.636945 94.116047) (width 0.25) (layer "B.Cu") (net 10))
 (segment (start 128.636945 98.054814) (end 127.5487 99.143058) (width 0.25) (layer "B.Cu") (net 10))
 (segment (start 127.5487 99.143058) (end 125.901456 99.143058) (width 0.25) (layer "B.Cu") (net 10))
 (segment (start 128.636945 94.116047) (end 128.636945 98.054814) (width 0.25) (layer "B.Cu") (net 10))
 (segment (start 125.901456 99.143058) (end 124.377425 97.619027) (width 0.25) (layer "B.Cu") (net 10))
 (segment (start 121.837425 92.539027) (end 126.917425 97.619027) (width 0.25) (layer "B.Cu") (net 11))
 (segment (start 121.837425 92.396527) (end 121.837425 92.539027) (width 0.25) (layer "B.Cu") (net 11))
 (segment (start 119.297425 81.429327) (end 109.137425 91.589327) (width 0.25) (layer "B.Cu") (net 4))
 (segment (start 109.137425 91.589327) (end 109.137425 97.619027) (width 0.25) (layer "B.Cu") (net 4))
 (segment (start 119.297425 77.156527) (end 119.297425 81.429327) (width 0.25) (layer "B.Cu") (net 4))
 (segment (start 124.377425 84.919027) (end 121.837425 87.459027) (width 0.25) (layer "F.Cu") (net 48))
 (segment (start 124.377425 77.156527) (end 124.377425 84.919027) (width 0.25) (layer "F.Cu") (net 48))
 (segment (start 129.457425 87.459027) (end 129.457425 92.396527) (width 0.25) (layer "F.Cu") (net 46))
 (segment (start 126.917425 82.379027) (end 126.917425 77.156527) (width 0.25) (layer "F.Cu") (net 47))
 (segment (start 116.757425 77.156527) (end 116.757425 82.379027) (width 0.25) (layer "F.Cu") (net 49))
 (segment (start 142.157425 87.459027) (end 142.157425 96.339027) (width 0.25) (layer "B.Cu") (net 19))
 (segment (start 142.157425 96.339027) (end 143.427425 97.609027) (width 0.25) (layer "B.Cu") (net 19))
 (segment (start 139.617425 96.339027) (end 140.887425 97.609027) (width 0.25) (layer "B.Cu") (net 18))
 (segment (start 139.617425 82.379027) (end 139.617425 96.339027) (width 0.25) (layer "B.Cu") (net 18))
 (segment (start 133.267425 72.209027) (end 138.347425 77.289027) (width 0.25) (layer "B.Cu") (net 17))
 (segment (start 138.347425 77.289027) (end 138.347425 97.609027) (width 0.25) (layer "B.Cu") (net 17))
 (segment (start 100.247425 83.639027) (end 100.247425 77.289027) (width 0.25) (layer "B.Cu") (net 17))
 (segment (start 104.067425 87.459027) (end 100.247425 83.639027) (width 0.25) (layer "B.Cu") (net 17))
 (segment (start 105.327425 72.209027) (end 133.267425 72.209027) (width 0.25) (layer "B.Cu") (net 17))
 (segment (start 109.137425 87.459027) (end 104.067425 87.459027) (width 0.25) (layer "B.Cu") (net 17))
 (segment (start 100.247425 77.289027) (end 105.327425 72.209027) (width 0.25) (layer "B.Cu") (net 17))
 (segment (start 113.777905 72.658547) (end 129.272662 72.658547) (width 0.25) (layer "B.Cu") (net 16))
 (segment (start 135.807425 88.573538) (end 133.267425 91.113538) (width 0.25) (layer "B.Cu") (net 16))
 (segment (start 104.057425 82.379027) (end 113.777905 72.658547) (width 0.25) (layer "B.Cu") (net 16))
 (segment (start 133.267425 95.069027) (end 135.807425 97.609027) (width 0.25) (layer "B.Cu") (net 16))
 (segment (start 133.267425 91.113538) (end 133.267425 95.069027) (width 0.25) (layer "B.Cu") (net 16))
 (segment (start 135.807425 79.19331) (end 135.807425 88.573538) (width 0.25) (layer "B.Cu") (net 16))
 (segment (start 129.272662 72.658547) (end 135.807425 79.19331) (width 0.25) (layer "B.Cu") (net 16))
 (segment (start 117.561636 113.983538) (end 137.212914 113.983538) (width 0.25) (layer "F.Cu") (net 41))
 (segment (start 137.212914 113.983538) (end 138.347425 112.849027) (width 0.25) (layer "F.Cu") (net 41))
 (segment (start 101.517425 110.319027) (end 113.897125 110.319027) (width 0.25) (layer "F.Cu") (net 41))
 (segment (start 113.897125 110.319027) (end 117.561636 113.983538) (width 0.25) (layer "F.Cu") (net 41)))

